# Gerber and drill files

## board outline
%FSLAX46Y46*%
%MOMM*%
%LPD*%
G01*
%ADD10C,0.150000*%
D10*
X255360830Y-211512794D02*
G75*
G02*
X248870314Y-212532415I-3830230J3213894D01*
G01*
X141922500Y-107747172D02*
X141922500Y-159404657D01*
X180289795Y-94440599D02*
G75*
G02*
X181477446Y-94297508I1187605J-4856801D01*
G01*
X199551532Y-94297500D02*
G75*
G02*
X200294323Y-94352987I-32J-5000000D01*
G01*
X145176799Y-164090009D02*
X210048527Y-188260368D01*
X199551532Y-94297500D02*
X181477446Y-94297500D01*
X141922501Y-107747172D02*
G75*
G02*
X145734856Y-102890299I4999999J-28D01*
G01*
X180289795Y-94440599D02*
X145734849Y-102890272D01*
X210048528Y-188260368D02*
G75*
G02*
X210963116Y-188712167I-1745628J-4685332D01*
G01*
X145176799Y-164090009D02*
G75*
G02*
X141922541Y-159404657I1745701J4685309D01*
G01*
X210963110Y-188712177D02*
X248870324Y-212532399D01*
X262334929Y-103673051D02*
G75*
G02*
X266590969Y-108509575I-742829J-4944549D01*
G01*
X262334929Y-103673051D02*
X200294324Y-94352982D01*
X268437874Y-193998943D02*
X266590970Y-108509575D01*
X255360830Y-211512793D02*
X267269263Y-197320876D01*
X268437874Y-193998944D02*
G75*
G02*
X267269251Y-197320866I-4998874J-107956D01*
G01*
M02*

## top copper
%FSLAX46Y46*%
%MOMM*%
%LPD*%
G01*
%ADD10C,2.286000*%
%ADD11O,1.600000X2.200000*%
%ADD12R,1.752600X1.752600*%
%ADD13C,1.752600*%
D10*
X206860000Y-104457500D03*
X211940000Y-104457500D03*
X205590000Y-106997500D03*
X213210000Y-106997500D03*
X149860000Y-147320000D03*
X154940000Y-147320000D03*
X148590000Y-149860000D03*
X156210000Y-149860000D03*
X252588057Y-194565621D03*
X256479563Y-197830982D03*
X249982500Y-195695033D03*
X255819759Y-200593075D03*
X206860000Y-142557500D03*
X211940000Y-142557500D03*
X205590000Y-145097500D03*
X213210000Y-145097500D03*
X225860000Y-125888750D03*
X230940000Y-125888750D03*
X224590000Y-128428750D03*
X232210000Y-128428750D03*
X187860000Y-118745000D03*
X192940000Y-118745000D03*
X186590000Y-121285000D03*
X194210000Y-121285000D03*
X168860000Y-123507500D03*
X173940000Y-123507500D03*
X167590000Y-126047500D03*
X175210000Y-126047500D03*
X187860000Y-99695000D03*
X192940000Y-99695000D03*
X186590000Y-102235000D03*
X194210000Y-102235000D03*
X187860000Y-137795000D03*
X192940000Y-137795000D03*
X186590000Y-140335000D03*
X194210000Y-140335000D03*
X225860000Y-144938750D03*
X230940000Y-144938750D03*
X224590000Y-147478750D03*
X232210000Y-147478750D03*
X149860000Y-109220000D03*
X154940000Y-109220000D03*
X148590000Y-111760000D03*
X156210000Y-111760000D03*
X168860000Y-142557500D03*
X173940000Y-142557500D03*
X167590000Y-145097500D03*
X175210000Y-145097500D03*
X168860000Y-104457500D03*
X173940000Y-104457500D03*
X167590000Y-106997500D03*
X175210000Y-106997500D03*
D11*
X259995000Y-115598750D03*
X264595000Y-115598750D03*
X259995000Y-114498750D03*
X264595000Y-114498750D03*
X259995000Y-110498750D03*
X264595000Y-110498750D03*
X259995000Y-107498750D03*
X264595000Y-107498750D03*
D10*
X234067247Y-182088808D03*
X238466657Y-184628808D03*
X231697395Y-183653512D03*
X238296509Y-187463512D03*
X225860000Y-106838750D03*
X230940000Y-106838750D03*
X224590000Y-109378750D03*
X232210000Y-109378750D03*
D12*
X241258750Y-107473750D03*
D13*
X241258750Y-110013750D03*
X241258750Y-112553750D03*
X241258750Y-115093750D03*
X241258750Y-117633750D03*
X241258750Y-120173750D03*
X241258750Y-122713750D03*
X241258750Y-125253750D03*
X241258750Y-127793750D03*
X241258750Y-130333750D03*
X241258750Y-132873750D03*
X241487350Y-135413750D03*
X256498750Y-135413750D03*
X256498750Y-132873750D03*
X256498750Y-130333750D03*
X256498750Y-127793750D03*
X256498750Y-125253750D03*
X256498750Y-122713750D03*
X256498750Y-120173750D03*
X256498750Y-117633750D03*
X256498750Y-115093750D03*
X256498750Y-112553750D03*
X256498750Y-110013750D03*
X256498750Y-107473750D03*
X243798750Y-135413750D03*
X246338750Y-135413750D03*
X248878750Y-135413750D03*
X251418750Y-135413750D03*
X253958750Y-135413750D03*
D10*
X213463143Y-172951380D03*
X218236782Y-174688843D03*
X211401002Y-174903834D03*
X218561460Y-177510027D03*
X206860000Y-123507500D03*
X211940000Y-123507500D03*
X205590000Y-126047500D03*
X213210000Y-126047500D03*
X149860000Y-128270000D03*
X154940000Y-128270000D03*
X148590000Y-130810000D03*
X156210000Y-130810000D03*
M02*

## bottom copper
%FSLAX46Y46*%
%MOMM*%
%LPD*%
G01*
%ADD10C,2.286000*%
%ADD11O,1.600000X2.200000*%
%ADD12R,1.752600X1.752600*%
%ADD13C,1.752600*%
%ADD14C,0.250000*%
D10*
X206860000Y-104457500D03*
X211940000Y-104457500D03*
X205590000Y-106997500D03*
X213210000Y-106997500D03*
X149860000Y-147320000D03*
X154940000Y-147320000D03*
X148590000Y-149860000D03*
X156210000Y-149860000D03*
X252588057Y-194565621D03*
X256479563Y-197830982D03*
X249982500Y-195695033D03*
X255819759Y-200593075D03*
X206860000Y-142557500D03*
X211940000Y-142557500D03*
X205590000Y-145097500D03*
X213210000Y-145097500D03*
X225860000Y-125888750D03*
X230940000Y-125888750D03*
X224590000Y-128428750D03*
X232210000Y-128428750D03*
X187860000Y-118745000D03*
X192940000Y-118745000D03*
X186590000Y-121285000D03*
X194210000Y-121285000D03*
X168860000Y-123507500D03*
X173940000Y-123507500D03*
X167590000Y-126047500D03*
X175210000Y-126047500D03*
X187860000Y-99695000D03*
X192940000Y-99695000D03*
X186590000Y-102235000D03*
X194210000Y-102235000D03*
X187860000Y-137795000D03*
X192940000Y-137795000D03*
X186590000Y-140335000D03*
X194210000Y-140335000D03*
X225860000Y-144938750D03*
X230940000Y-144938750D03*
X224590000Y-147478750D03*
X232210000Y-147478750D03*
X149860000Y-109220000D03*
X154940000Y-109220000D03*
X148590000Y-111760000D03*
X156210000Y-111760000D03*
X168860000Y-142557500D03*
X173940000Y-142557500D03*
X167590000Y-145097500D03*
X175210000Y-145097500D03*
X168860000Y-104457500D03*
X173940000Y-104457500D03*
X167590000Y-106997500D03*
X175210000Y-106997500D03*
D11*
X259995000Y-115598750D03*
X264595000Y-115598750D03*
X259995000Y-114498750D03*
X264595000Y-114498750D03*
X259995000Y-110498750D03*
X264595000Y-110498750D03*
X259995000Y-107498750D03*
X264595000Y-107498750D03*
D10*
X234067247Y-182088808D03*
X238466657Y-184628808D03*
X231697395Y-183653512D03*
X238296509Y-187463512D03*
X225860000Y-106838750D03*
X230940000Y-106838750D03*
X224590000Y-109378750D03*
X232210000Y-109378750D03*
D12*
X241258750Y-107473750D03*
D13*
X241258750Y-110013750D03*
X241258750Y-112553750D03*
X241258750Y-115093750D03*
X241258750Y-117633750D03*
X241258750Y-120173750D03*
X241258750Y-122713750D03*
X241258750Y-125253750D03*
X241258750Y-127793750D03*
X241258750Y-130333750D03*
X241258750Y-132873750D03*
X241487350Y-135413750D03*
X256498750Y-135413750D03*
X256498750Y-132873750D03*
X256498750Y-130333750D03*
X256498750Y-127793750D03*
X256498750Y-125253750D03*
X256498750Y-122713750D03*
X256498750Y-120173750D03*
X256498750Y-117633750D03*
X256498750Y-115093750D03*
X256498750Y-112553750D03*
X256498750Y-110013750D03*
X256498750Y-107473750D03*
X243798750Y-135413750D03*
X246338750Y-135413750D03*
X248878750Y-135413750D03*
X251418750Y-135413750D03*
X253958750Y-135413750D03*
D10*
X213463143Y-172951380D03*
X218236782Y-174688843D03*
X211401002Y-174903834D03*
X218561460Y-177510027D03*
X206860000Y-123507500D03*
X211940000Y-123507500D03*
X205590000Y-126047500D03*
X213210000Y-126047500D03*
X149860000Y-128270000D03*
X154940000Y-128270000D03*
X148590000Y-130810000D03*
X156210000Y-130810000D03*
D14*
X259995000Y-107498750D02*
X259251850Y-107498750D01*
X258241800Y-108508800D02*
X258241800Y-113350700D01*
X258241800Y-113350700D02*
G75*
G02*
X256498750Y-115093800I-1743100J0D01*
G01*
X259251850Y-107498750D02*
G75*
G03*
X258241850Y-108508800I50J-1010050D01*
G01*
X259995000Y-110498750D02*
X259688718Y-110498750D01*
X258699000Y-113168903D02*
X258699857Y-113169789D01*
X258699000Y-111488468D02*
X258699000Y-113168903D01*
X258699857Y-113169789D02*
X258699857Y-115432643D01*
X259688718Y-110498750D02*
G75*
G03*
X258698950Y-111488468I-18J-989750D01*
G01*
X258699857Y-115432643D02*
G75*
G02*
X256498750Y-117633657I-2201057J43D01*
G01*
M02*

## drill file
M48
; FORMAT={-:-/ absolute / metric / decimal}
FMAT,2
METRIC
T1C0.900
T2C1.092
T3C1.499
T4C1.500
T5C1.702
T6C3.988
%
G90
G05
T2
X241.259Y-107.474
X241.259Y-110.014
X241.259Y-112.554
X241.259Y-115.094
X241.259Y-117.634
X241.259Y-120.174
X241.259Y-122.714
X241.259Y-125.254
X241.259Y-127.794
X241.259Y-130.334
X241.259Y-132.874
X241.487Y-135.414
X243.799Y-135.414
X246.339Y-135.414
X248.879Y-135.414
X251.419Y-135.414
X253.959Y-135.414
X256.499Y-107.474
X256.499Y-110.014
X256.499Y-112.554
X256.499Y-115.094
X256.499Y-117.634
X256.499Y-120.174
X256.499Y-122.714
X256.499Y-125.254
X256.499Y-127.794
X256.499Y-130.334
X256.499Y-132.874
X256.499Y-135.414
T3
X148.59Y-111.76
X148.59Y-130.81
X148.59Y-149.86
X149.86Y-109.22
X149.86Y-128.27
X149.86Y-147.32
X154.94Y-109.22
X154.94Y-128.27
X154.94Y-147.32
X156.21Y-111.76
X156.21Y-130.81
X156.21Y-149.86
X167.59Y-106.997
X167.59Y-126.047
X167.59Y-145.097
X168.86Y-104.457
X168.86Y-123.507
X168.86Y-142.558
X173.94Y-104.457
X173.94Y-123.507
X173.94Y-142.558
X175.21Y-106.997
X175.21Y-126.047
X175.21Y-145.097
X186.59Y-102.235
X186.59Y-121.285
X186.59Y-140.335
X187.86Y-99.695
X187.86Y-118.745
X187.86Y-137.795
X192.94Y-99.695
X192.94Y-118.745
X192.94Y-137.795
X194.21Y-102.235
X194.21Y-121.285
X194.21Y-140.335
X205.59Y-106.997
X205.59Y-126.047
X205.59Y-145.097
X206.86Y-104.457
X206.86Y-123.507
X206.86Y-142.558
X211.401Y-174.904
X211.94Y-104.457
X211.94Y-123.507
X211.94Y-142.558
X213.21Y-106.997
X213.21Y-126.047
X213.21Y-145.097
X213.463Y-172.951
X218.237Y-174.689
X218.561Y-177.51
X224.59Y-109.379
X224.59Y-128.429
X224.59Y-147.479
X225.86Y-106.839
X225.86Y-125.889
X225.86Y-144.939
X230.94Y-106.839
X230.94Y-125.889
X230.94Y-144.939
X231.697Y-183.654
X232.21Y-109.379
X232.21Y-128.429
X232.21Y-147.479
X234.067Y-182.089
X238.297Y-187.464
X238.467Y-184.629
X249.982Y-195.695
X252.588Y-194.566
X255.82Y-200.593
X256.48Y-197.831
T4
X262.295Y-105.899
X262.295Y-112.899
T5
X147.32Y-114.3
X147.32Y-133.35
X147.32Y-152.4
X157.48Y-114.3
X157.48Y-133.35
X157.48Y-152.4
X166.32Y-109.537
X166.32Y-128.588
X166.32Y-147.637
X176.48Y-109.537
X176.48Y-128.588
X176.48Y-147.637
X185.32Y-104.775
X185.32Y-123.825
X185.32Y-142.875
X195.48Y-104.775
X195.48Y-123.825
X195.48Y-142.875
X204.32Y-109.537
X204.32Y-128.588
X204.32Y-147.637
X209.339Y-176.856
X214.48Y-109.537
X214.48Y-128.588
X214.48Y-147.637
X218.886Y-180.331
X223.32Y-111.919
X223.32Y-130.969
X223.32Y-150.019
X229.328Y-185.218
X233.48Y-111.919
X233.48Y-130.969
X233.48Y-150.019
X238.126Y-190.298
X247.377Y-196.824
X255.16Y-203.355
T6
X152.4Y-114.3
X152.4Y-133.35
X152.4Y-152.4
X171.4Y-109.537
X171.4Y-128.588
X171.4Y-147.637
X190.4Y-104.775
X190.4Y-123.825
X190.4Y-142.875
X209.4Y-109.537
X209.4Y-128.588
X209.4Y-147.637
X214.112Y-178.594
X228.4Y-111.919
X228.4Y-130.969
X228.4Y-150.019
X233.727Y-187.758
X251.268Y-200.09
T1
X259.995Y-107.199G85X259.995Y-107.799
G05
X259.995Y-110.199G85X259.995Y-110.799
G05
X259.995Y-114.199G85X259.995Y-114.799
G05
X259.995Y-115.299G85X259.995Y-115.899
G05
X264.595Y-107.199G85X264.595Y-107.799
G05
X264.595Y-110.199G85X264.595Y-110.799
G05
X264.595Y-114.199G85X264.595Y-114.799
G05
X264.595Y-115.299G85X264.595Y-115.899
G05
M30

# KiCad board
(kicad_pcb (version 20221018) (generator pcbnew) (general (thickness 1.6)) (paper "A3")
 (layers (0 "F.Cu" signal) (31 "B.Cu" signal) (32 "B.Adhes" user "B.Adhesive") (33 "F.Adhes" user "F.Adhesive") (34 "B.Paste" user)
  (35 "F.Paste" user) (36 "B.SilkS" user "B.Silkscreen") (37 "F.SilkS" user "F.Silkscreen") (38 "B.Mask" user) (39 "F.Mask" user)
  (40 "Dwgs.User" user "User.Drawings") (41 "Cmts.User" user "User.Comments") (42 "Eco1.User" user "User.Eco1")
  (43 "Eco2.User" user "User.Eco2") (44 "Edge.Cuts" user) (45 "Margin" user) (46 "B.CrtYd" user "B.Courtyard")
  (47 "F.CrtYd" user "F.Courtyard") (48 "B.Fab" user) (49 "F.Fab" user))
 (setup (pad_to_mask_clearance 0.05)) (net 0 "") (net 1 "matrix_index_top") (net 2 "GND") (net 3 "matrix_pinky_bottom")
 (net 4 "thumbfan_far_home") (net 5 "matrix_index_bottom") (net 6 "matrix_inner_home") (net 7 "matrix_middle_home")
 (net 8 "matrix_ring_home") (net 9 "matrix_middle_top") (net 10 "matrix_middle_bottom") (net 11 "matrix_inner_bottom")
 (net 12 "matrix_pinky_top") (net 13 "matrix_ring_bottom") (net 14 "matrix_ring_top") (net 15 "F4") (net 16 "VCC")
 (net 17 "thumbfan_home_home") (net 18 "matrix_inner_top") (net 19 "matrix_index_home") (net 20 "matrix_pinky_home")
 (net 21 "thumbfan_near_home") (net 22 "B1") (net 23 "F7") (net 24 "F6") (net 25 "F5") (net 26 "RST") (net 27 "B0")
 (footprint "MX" (layer "F.Cu") (at 209.4 109.5375)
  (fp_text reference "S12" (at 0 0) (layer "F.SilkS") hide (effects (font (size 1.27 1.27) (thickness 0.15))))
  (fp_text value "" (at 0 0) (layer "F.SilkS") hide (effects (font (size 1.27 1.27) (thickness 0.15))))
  (pad "" np_thru_hole circle (at -5.08 0) (size 1.7018 1.7018) (drill 1.7018) (layers "*.Cu" "*.Mask"))
  (pad "" np_thru_hole circle (at 0 0) (size 3.9878 3.9878) (drill 3.9878) (layers "*.Cu" "*.Mask"))
  (pad "" np_thru_hole circle (at 5.08 0) (size 1.7018 1.7018) (drill 1.7018) (layers "*.Cu" "*.Mask"))
  (pad "1" thru_hole circle (at -2.54 -5.08) (size 2.286 2.286) (drill 1.4986) (layers "*.Cu" "*.Mask") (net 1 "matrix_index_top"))
  (pad "1" thru_hole circle (at 2.54 -5.08) (size 2.286 2.286) (drill 1.4986) (layers "*.Cu" "*.Mask") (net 1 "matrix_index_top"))
  (pad "2" thru_hole circle (at -3.81 -2.54) (size 2.286 2.286) (drill 1.4986) (layers "*.Cu" "*.Mask") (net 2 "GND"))
  (pad "2" thru_hole circle (at 3.81 -2.54) (size 2.286 2.286) (drill 1.4986) (layers "*.Cu" "*.Mask") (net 2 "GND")))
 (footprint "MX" (layer "F.Cu") (at 152.4 152.4)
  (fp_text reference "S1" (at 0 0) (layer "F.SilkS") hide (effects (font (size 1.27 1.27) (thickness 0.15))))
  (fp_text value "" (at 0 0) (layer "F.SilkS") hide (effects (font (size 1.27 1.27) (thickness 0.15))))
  (pad "" np_thru_hole circle (at -5.08 0) (size 1.7018 1.7018) (drill 1.7018) (layers "*.Cu" "*.Mask"))
  (pad "" np_thru_hole circle (at 0 0) (size 3.9878 3.9878) (drill 3.9878) (layers "*.Cu" "*.Mask"))
  (pad "" np_thru_hole circle (at 5.08 0) (size 1.7018 1.7018) (drill 1.7018) (layers "*.Cu" "*.Mask"))
  (pad "1" thru_hole circle (at -2.54 -5.08) (size 2.286 2.286) (drill 1.4986) (layers "*.Cu" "*.Mask") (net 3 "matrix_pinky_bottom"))
  (pad "1" thru_hole circle (at 2.54 -5.08) (size 2.286 2.286) (drill 1.4986) (layers "*.Cu" "*.Mask") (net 3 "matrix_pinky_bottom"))
  (pad "2" thru_hole circle (at -3.81 -2.54) (size 2.286 2.286) (drill 1.4986) (layers "*.Cu" "*.Mask") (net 2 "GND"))
  (pad "2" thru_hole circle (at 3.81 -2.54) (size 2.286 2.286) (drill 1.4986) (layers "*.Cu" "*.Mask") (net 2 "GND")))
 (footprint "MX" (layer "F.Cu") (at 251.268449 200.089807 -40)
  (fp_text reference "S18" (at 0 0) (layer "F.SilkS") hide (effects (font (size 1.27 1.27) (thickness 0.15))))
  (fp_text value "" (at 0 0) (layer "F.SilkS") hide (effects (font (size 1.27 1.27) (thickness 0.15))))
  (pad "" np_thru_hole circle (at -5.08 0) (size 1.7018 1.7018) (drill 1.7018) (layers "*.Cu" "*.Mask"))
  (pad "" np_thru_hole circle (at 0 0) (size 3.9878 3.9878) (drill 3.9878) (layers "*.Cu" "*.Mask"))
  (pad "" np_thru_hole circle (at 5.08 0) (size 1.7018 1.7018) (drill 1.7018) (layers "*.Cu" "*.Mask"))
  (pad "1" thru_hole circle (at -2.54 -5.08) (size 2.286 2.286) (drill 1.4986) (layers "*.Cu" "*.Mask") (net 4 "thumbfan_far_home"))
  (pad "1" thru_hole circle (at 2.54 -5.08) (size 2.286 2.286) (drill 1.4986) (layers "*.Cu" "*.Mask") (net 4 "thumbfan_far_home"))
  (pad "2" thru_hole circle (at -3.81 -2.54) (size 2.286 2.286) (drill 1.4986) (layers "*.Cu" "*.Mask") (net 2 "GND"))
  (pad "2" thru_hole circle (at 3.81 -2.54) (size 2.286 2.286) (drill 1.4986) (layers "*.Cu" "*.Mask") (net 2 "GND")))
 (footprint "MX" (layer "F.Cu") (at 209.4 147.6375)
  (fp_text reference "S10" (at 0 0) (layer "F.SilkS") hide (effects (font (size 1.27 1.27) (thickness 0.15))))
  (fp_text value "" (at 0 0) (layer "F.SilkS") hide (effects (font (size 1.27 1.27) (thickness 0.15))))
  (pad "" np_thru_hole circle (at -5.08 0) (size 1.7018 1.7018) (drill 1.7018) (layers "*.Cu" "*.Mask"))
  (pad "" np_thru_hole circle (at 0 0) (size 3.9878 3.9878) (drill 3.9878) (layers "*.Cu" "*.Mask"))
  (pad "" np_thru_hole circle (at 5.08 0) (size 1.7018 1.7018) (drill 1.7018) (layers "*.Cu" "*.Mask"))
  (pad "1" thru_hole circle (at -2.54 -5.08) (size 2.286 2.286) (drill 1.4986) (layers "*.Cu" "*.Mask") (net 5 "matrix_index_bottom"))
  (pad "1" thru_hole circle (at 2.54 -5.08) (size 2.286 2.286) (drill 1.4986) (layers "*.Cu" "*.Mask") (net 5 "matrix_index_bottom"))
  (pad "2" thru_hole circle (at -3.81 -2.54) (size 2.286 2.286) (drill 1.4986) (layers "*.Cu" "*.Mask") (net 2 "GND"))
  (pad "2" thru_hole circle (at 3.81 -2.54) (size 2.286 2.286) (drill 1.4986) (layers "*.Cu" "*.Mask") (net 2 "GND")))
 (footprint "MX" (layer "F.Cu") (at 228.4 130.96875)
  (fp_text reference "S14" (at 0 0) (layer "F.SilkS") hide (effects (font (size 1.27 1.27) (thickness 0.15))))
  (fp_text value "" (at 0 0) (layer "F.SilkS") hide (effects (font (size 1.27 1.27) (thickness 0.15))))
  (pad "" np_thru_hole circle (at -5.08 0) (size 1.7018 1.7018) (drill 1.7018) (layers "*.Cu" "*.Mask"))
  (pad "" np_thru_hole circle (at 0 0) (size 3.9878 3.9878) (drill 3.9878) (layers "*.Cu" "*.Mask"))
  (pad "" np_thru_hole circle (at 5.08 0) (size 1.7018 1.7018) (drill 1.7018) (layers "*.Cu" "*.Mask"))
  (pad "1" thru_hole circle (at -2.54 -5.08) (size 2.286 2.286) (drill 1.4986) (layers "*.Cu" "*.Mask") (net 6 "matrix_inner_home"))
  (pad "1" thru_hole circle (at 2.54 -5.08) (size 2.286 2.286) (drill 1.4986) (layers "*.Cu" "*.Mask") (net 6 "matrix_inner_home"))
  (pad "2" thru_hole circle (at -3.81 -2.54) (size 2.286 2.286) (drill 1.4986) (layers "*.Cu" "*.Mask") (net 2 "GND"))
  (pad "2" thru_hole circle (at 3.81 -2.54) (size 2.286 2.286) (drill 1.4986) (layers "*.Cu" "*.Mask") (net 2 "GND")))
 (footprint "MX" (layer "F.Cu") (at 190.4 123.825)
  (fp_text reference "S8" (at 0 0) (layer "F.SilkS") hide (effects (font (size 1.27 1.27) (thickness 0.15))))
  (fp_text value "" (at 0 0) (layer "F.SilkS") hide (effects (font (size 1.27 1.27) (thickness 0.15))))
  (pad "" np_thru_hole circle (at -5.08 0) (size 1.7018 1.7018) (drill 1.7018) (layers "*.Cu" "*.Mask"))
  (pad "" np_thru_hole circle (at 0 0) (size 3.9878 3.9878) (drill 3.9878) (layers "*.Cu" "*.Mask"))
  (pad "" np_thru_hole circle (at 5.08 0) (size 1.7018 1.7018) (drill 1.7018) (layers "*.Cu" "*.Mask"))
  (pad "1" thru_hole circle (at -2.54 -5.08) (size 2.286 2.286) (drill 1.4986) (layers "*.Cu" "*.Mask") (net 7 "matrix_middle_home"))
  (pad "1" thru_hole circle (at 2.54 -5.08) (size 2.286 2.286) (drill 1.4986) (layers "*.Cu" "*.Mask") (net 7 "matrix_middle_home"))
  (pad "2" thru_hole circle (at -3.81 -2.54) (size 2.286 2.286) (drill 1.4986) (layers "*.Cu" "*.Mask") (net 2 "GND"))
  (pad "2" thru_hole circle (at 3.81 -2.54) (size 2.286 2.286) (drill 1.4986) (layers "*.Cu" "*.Mask") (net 2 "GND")))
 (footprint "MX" (layer "F.Cu") (at 171.4 128.5875)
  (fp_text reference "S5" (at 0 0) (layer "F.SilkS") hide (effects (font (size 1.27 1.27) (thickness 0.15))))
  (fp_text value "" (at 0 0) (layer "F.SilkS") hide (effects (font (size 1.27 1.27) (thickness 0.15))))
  (pad "" np_thru_hole circle (at -5.08 0) (size 1.7018 1.7018) (drill 1.7018) (layers "*.Cu" "*.Mask"))
  (pad "" np_thru_hole circle (at 0 0) (size 3.9878 3.9878) (drill 3.9878) (layers "*.Cu" "*.Mask"))
  (pad "" np_thru_hole circle (at 5.08 0) (size 1.7018 1.7018) (drill 1.7018) (layers "*.Cu" "*.Mask"))
  (pad "1" thru_hole circle (at -2.54 -5.08) (size 2.286 2.286) (drill 1.4986) (layers "*.Cu" "*.Mask") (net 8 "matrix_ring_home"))
  (pad "1" thru_hole circle (at 2.54 -5.08) (size 2.286 2.286) (drill 1.4986) (layers "*.Cu" "*.Mask") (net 8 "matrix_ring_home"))
  (pad "2" thru_hole circle (at -3.81 -2.54) (size 2.286 2.286) (drill 1.4986) (layers "*.Cu" "*.Mask") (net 2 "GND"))
  (pad "2" thru_hole circle (at 3.81 -2.54) (size 2.286 2.286) (drill 1.4986) (layers "*.Cu" "*.Mask") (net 2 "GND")))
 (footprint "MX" (layer "F.Cu") (at 190.4 104.775)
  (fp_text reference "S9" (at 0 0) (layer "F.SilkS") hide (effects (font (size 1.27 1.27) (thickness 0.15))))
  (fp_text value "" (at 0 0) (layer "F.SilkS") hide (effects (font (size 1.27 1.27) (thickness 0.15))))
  (pad "" np_thru_hole circle (at -5.08 0) (size 1.7018 1.7018) (drill 1.7018) (layers "*.Cu" "*.Mask"))
  (pad "" np_thru_hole circle (at 0 0) (size 3.9878 3.9878) (drill 3.9878) (layers "*.Cu" "*.Mask"))
  (pad "" np_thru_hole circle (at 5.08 0) (size 1.7018 1.7018) (drill 1.7018) (layers "*.Cu" "*.Mask"))
  (pad "1" thru_hole circle (at -2.54 -5.08) (size 2.286 2.286) (drill 1.4986) (layers "*.Cu" "*.Mask") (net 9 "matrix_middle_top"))
  (pad "1" thru_hole circle (at 2.54 -5.08) (size 2.286 2.286) (drill 1.4986) (layers "*.Cu" "*.Mask") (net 9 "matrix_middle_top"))
  (pad "2" thru_hole circle (at -3.81 -2.54) (size 2.286 2.286) (drill 1.4986) (layers "*.Cu" "*.Mask") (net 2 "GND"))
  (pad "2" thru_hole circle (at 3.81 -2.54) (size 2.286 2.286) (drill 1.4986) (layers "*.Cu" "*.Mask") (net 2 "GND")))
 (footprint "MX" (layer "F.Cu") (at 190.4 142.875)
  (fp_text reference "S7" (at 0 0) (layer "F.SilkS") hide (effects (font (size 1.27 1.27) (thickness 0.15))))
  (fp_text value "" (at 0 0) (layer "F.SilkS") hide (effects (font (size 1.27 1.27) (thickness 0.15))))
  (pad "" np_thru_hole circle (at -5.08 0) (size 1.7018 1.7018) (drill 1.7018) (layers "*.Cu" "*.Mask"))
  (pad "" np_thru_hole circle (at 0 0) (size 3.9878 3.9878) (drill 3.9878) (layers "*.Cu" "*.Mask"))
  (pad "" np_thru_hole circle (at 5.08 0) (size 1.7018 1.7018) (drill 1.7018) (layers "*.Cu" "*.Mask"))
  (pad "1" thru_hole circle (at -2.54 -5.08) (size 2.286 2.286) (drill 1.4986) (layers "*.Cu" "*.Mask") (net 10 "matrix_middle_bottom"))
  (pad "1" thru_hole circle (at 2.54 -5.08) (size 2.286 2.286) (drill 1.4986) (layers "*.Cu" "*.Mask") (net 10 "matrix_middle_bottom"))
  (pad "2" thru_hole circle (at -3.81 -2.54) (size 2.286 2.286) (drill 1.4986) (layers "*.Cu" "*.Mask") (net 2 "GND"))
  (pad "2" thru_hole circle (at 3.81 -2.54) (size 2.286 2.286) (drill 1.4986) (layers "*.Cu" "*.Mask") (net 2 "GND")))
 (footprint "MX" (layer "F.Cu") (at 228.4 150.01875)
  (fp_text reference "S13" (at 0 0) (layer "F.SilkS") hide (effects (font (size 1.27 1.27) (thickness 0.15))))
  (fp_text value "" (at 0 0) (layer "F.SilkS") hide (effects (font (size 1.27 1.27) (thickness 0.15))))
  (pad "" np_thru_hole circle (at -5.08 0) (size 1.7018 1.7018) (drill 1.7018) (layers "*.Cu" "*.Mask"))
  (pad "" np_thru_hole circle (at 0 0) (size 3.9878 3.9878) (drill 3.9878) (layers "*.Cu" "*.Mask"))
  (pad "" np_thru_hole circle (at 5.08 0) (size 1.7018 1.7018) (drill 1.7018) (layers "*.Cu" "*.Mask"))
  (pad "1" thru_hole circle (at -2.54 -5.08) (size 2.286 2.286) (drill 1.4986) (layers "*.Cu" "*.Mask") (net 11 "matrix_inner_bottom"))
  (pad "1" thru_hole circle (at 2.54 -5.08) (size 2.286 2.286) (drill 1.4986) (layers "*.Cu" "*.Mask") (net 11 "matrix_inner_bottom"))
  (pad "2" thru_hole circle (at -3.81 -2.54) (size 2.286 2.286) (drill 1.4986) (layers "*.Cu" "*.Mask") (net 2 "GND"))
  (pad "2" thru_hole circle (at 3.81 -2.54) (size 2.286 2.286) (drill 1.4986) (layers "*.Cu" "*.Mask") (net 2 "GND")))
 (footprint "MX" (layer "F.Cu") (at 152.4 114.3)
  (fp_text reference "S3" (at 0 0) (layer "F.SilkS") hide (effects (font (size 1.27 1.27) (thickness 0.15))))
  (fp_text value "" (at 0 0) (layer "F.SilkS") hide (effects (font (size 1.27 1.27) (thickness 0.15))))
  (pad "" np_thru_hole circle (at -5.08 0) (size 1.7018 1.7018) (drill 1.7018) (layers "*.Cu" "*.Mask"))
  (pad "" np_thru_hole circle (at 0 0) (size 3.9878 3.9878) (drill 3.9878) (layers "*.Cu" "*.Mask"))
  (pad "" np_thru_hole circle (at 5.08 0) (size 1.7018 1.7018) (drill 1.7018) (layers "*.Cu" "*.Mask"))
  (pad "1" thru_hole circle (at -2.54 -5.08) (size 2.286 2.286) (drill 1.4986) (layers "*.Cu" "*.Mask") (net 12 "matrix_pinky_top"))
  (pad "1" thru_hole circle (at 2.54 -5.08) (size 2.286 2.286) (drill 1.4986) (layers "*.Cu" "*.Mask") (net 12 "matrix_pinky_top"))
  (pad "2" thru_hole circle (at -3.81 -2.54) (size 2.286 2.286) (drill 1.4986) (layers "*.Cu" "*.Mask") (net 2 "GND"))
  (pad "2" thru_hole circle (at 3.81 -2.54) (size 2.286 2.286) (drill 1.4986) (layers "*.Cu" "*.Mask") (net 2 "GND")))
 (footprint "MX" (layer "F.Cu") (at 171.4 147.6375)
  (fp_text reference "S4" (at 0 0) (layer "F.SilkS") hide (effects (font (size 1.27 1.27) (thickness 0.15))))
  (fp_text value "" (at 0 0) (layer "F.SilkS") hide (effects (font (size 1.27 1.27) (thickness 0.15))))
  (pad "" np_thru_hole circle (at -5.08 0) (size 1.7018 1.7018) (drill 1.7018) (layers "*.Cu" "*.Mask"))
  (pad "" np_thru_hole circle (at 0 0) (size 3.9878 3.9878) (drill 3.9878) (layers "*.Cu" "*.Mask"))
  (pad "" np_thru_hole circle (at 5.08 0) (size 1.7018 1.7018) (drill 1.7018) (layers "*.Cu" "*.Mask"))
  (pad "1" thru_hole circle (at -2.54 -5.08) (size 2.286 2.286) (drill 1.4986) (layers "*.Cu" "*.Mask") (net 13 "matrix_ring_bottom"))
  (pad "1" thru_hole circle (at 2.54 -5.08) (size 2.286 2.286) (drill 1.4986) (layers "*.Cu" "*.Mask") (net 13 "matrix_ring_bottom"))
  (pad "2" thru_hole circle (at -3.81 -2.54) (size 2.286 2.286) (drill 1.4986) (layers "*.Cu" "*.Mask") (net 2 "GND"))
  (pad "2" thru_hole circle (at 3.81 -2.54) (size 2.286 2.286) (drill 1.4986) (layers "*.Cu" "*.Mask") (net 2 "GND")))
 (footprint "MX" (layer "F.Cu") (at 171.4 109.5375)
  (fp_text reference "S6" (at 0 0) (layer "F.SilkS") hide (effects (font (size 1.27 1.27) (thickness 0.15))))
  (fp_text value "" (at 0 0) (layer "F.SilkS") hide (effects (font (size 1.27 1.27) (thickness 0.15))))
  (pad "" np_thru_hole circle (at -5.08 0) (size 1.7018 1.7018) (drill 1.7018) (layers "*.Cu" "*.Mask"))
  (pad "" np_thru_hole circle (at 0 0) (size 3.9878 3.9878) (drill 3.9878) (layers "*.Cu" "*.Mask"))
  (pad "" np_thru_hole circle (at 5.08 0) (size 1.7018 1.7018) (drill 1.7018) (layers "*.Cu" "*.Mask"))
  (pad "1" thru_hole circle (at -2.54 -5.08) (size 2.286 2.286) (drill 1.4986) (layers "*.Cu" "*.Mask") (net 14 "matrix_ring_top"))
  (pad "1" thru_hole circle (at 2.54 -5.08) (size 2.286 2.286) (drill 1.4986) (layers "*.Cu" "*.Mask") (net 14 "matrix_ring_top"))
  (pad "2" thru_hole circle (at -3.81 -2.54) (size 2.286 2.286) (drill 1.4986) (layers "*.Cu" "*.Mask") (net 2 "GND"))
  (pad "2" thru_hole circle (at 3.81 -2.54) (size 2.286 2.286) (drill 1.4986) (layers "*.Cu" "*.Mask") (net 2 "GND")))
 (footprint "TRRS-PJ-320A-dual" (layer "F.Cu") (at 264.595 104.29875)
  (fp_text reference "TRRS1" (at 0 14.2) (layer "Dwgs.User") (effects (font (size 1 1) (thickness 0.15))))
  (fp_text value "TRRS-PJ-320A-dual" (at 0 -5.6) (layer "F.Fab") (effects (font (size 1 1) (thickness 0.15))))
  (pad "" np_thru_hole circle (at -2.3 1.6) (size 1.5 1.5) (drill 1.5) (layers "*.Cu" "*.Mask"))
  (pad "" np_thru_hole circle (at -2.3 8.6) (size 1.5 1.5) (drill 1.5) (layers "*.Cu" "*.Mask"))
  (pad "1" thru_hole oval (at -4.6 11.3) (size 1.6 2.2) (drill oval 0.9 1.5) (layers "*.Cu" "*.Mask") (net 2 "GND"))
  (pad "1" thru_hole oval (at 0 11.3) (size 1.6 2.2) (drill oval 0.9 1.5) (layers "*.Cu" "*.Mask") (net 2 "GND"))
  (pad "2" thru_hole oval (at -4.6 10.2) (size 1.6 2.2) (drill oval 0.9 1.5) (layers "*.Cu" "*.Mask") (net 2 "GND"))
  (pad "2" thru_hole oval (at 0 10.2) (size 1.6 2.2) (drill oval 0.9 1.5) (layers "*.Cu" "*.Mask") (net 2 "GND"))
  (pad "3" thru_hole oval (at -4.6 6.2) (size 1.6 2.2) (drill oval 0.9 1.5) (layers "*.Cu" "*.Mask") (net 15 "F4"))
  (pad "3" thru_hole oval (at 0 6.2) (size 1.6 2.2) (drill oval 0.9 1.5) (layers "*.Cu" "*.Mask") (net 15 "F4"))
  (pad "4" thru_hole oval (at -4.6 3.2) (size 1.6 2.2) (drill oval 0.9 1.5) (layers "*.Cu" "*.Mask") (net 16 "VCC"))
  (pad "4" thru_hole oval (at 0 3.2) (size 1.6 2.2) (drill oval 0.9 1.5) (layers "*.Cu" "*.Mask") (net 16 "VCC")))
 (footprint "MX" (layer "F.Cu") (at 233.726952 187.758217 -30)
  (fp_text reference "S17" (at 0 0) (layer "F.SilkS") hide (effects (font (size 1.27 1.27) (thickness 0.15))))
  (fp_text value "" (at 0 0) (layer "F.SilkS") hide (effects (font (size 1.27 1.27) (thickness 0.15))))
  (pad "" np_thru_hole circle (at -5.08 0) (size 1.7018 1.7018) (drill 1.7018) (layers "*.Cu" "*.Mask"))
  (pad "" np_thru_hole circle (at 0 0) (size 3.9878 3.9878) (drill 3.9878) (layers "*.Cu" "*.Mask"))
  (pad "" np_thru_hole circle (at 5.08 0) (size 1.7018 1.7018) (drill 1.7018) (layers "*.Cu" "*.Mask"))
  (pad "1" thru_hole circle (at -2.54 -5.08) (size 2.286 2.286) (drill 1.4986) (layers "*.Cu" "*.Mask") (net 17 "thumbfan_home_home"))
  (pad "1" thru_hole circle (at 2.54 -5.08) (size 2.286 2.286) (drill 1.4986) (layers "*.Cu" "*.Mask") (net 17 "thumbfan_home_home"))
  (pad "2" thru_hole circle (at -3.81 -2.54) (size 2.286 2.286) (drill 1.4986) (layers "*.Cu" "*.Mask") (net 2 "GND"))
  (pad "2" thru_hole circle (at 3.81 -2.54) (size 2.286 2.286) (drill 1.4986) (layers "*.Cu" "*.Mask") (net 2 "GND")))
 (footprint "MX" (layer "F.Cu") (at 228.4 111.91875)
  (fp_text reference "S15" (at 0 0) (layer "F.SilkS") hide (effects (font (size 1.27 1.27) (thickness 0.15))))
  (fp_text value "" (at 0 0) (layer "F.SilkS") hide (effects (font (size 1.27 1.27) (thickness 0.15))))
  (pad "" np_thru_hole circle (at -5.08 0) (size 1.7018 1.7018) (drill 1.7018) (layers "*.Cu" "*.Mask"))
  (pad "" np_thru_hole circle (at 0 0) (size 3.9878 3.9878) (drill 3.9878) (layers "*.Cu" "*.Mask"))
  (pad "" np_thru_hole circle (at 5.08 0) (size 1.7018 1.7018) (drill 1.7018) (layers "*.Cu" "*.Mask"))
  (pad "1" thru_hole circle (at -2.54 -5.08) (size 2.286 2.286) (drill 1.4986) (layers "*.Cu" "*.Mask") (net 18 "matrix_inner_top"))
  (pad "1" thru_hole circle (at 2.54 -5.08) (size 2.286 2.286) (drill 1.4986) (layers "*.Cu" "*.Mask") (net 18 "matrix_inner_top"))
  (pad "2" thru_hole circle (at -3.81 -2.54) (size 2.286 2.286) (drill 1.4986) (layers "*.Cu" "*.Mask") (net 2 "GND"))
  (pad "2" thru_hole circle (at 3.81 -2.54) (size 2.286 2.286) (drill 1.4986) (layers "*.Cu" "*.Mask") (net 2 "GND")))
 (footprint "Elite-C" (layer "F.Cu") (at 248.87875 121.44375 -90)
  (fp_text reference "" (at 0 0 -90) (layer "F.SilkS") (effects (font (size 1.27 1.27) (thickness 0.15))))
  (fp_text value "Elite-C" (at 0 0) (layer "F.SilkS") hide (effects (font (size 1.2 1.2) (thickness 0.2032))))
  (pad "1" thru_hole rect (at -13.97 7.62) (size 1.7526 1.7526) (drill 1.0922) (layers "*.Cu" "*.SilkS" "*.Mask")
   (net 18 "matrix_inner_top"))
  (pad "2" thru_hole circle (at -11.43 7.62) (size 1.7526 1.7526) (drill 1.0922) (layers "*.Cu" "*.SilkS" "*.Mask")
   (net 1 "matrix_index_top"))
  (pad "3" thru_hole circle (at -8.89 7.62) (size 1.7526 1.7526) (drill 1.0922) (layers "*.Cu" "*.SilkS" "*.Mask") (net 2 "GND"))
  (pad "4" thru_hole circle (at -6.35 7.62) (size 1.7526 1.7526) (drill 1.0922) (layers "*.Cu" "*.SilkS" "*.Mask") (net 2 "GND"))
  (pad "5" thru_hole circle (at -3.81 7.62) (size 1.7526 1.7526) (drill 1.0922) (layers "*.Cu" "*.SilkS" "*.Mask")
   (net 9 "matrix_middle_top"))
  (pad "6" thru_hole circle (at -1.27 7.62) (size 1.7526 1.7526) (drill 1.0922) (layers "*.Cu" "*.SilkS" "*.Mask")
   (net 14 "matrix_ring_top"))
  (pad "7" thru_hole circle (at 1.27 7.62) (size 1.7526 1.7526) (drill 1.0922) (layers "*.Cu" "*.SilkS" "*.Mask")
   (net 12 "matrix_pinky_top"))
  (pad "8" thru_hole circle (at 3.81 7.62) (size 1.7526 1.7526) (drill 1.0922) (layers "*.Cu" "*.SilkS" "*.Mask")
   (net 7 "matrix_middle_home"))
  (pad "9" thru_hole circle (at 6.35 7.62) (size 1.7526 1.7526) (drill 1.0922) (layers "*.Cu" "*.SilkS" "*.Mask")
   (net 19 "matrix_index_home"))
  (pad "10" thru_hole circle (at 8.89 7.62) (size 1.7526 1.7526) (drill 1.0922) (layers "*.Cu" "*.SilkS" "*.Mask")
   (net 6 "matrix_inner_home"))
  (pad "11" thru_hole circle (at 11.43 7.62) (size 1.7526 1.7526) (drill 1.0922) (layers "*.Cu" "*.SilkS" "*.Mask")
   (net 8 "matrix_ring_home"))
  (pad "12" thru_hole circle (at 13.97 7.3914) (size 1.7526 1.7526) (drill 1.0922) (layers "*.Cu" "*.SilkS" "*.Mask")
   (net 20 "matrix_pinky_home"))
  (pad "13" thru_hole circle (at 13.97 -7.62) (size 1.7526 1.7526) (drill 1.0922) (layers "*.Cu" "*.SilkS" "*.Mask")
   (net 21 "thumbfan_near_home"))
  (pad "14" thru_hole circle (at 11.43 -7.62) (size 1.7526 1.7526) (drill 1.0922) (layers "*.Cu" "*.SilkS" "*.Mask")
   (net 17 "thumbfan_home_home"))
  (pad "15" thru_hole circle (at 8.89 -7.62) (size 1.7526 1.7526) (drill 1.0922) (layers "*.Cu" "*.SilkS" "*.Mask")
   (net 4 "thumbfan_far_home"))
  (pad "16" thru_hole circle (at 6.35 -7.62) (size 1.7526 1.7526) (drill 1.0922) (layers "*.Cu" "*.SilkS" "*.Mask") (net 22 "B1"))
  (pad "17" thru_hole circle (at 3.81 -7.62) (size 1.7526 1.7526) (drill 1.0922) (layers "*.Cu" "*.SilkS" "*.Mask") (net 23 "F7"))
  (pad "18" thru_hole circle (at 1.27 -7.62) (size 1.7526 1.7526) (drill 1.0922) (layers "*.Cu" "*.SilkS" "*.Mask") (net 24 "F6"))
  (pad "19" thru_hole circle (at -1.27 -7.62) (size 1.7526 1.7526) (drill 1.0922) (layers "*.Cu" "*.SilkS" "*.Mask") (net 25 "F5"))
  (pad "20" thru_hole circle (at -3.81 -7.62) (size 1.7526 1.7526) (drill 1.0922) (layers "*.Cu" "*.SilkS" "*.Mask") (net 15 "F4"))
  (pad "21" thru_hole circle (at -6.35 -7.62) (size 1.7526 1.7526) (drill 1.0922) (layers "*.Cu" "*.SilkS" "*.Mask") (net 16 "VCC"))
  (pad "22" thru_hole circle (at -8.89 -7.62) (size 1.7526 1.7526) (drill 1.0922) (layers "*.Cu" "*.SilkS" "*.Mask") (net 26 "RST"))
  (pad "23" thru_hole circle (at -11.43 -7.62) (size 1.7526 1.7526) (drill 1.0922) (layers "*.Cu" "*.SilkS" "*.Mask") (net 2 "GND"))
  (pad "24" thru_hole circle (at -13.97 -7.62) (size 1.7526 1.7526) (drill 1.0922) (layers "*.Cu" "*.SilkS" "*.Mask") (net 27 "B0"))
  (pad "25" thru_hole circle (at 13.97 5.08) (size 1.7526 1.7526) (drill 1.0922) (layers "*.Cu" "*.SilkS" "*.Mask")
   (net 10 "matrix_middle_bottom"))
  (pad "26" thru_hole circle (at 13.97 2.54) (size 1.7526 1.7526) (drill 1.0922) (layers "*.Cu" "*.SilkS" "*.Mask")
   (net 5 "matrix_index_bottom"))
  (pad "27" thru_hole circle (at 13.97 0) (size 1.7526 1.7526) (drill 1.0922) (layers "*.Cu" "*.SilkS" "*.Mask")
   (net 11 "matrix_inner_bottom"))
  (pad "28" thru_hole circle (at 13.97 -2.54) (size 1.7526 1.7526) (drill 1.0922) (layers "*.Cu" "*.SilkS" "*.Mask")
   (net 3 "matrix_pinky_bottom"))
  (pad "29" thru_hole circle (at 13.97 -5.08) (size 1.7526 1.7526) (drill 1.0922) (layers "*.Cu" "*.SilkS" "*.Mask")
   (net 13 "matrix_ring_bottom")))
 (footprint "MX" (layer "F.Cu") (at 214.1125 178.59375 -20)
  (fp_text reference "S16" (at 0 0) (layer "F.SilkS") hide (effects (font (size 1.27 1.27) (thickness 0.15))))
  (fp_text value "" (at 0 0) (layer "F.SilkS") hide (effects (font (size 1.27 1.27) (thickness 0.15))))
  (pad "" np_thru_hole circle (at -5.08 0) (size 1.7018 1.7018) (drill 1.7018) (layers "*.Cu" "*.Mask"))
  (pad "" np_thru_hole circle (at 0 0) (size 3.9878 3.9878) (drill 3.9878) (layers "*.Cu" "*.Mask"))
  (pad "" np_thru_hole circle (at 5.08 0) (size 1.7018 1.7018) (drill 1.7018) (layers "*.Cu" "*.Mask"))
  (pad "1" thru_hole circle (at -2.54 -5.08) (size 2.286 2.286) (drill 1.4986) (layers "*.Cu" "*.Mask") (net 21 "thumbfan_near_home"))
  (pad "1" thru_hole circle (at 2.54 -5.08) (size 2.286 2.286) (drill 1.4986) (layers "*.Cu" "*.Mask") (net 21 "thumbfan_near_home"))
  (pad "2" thru_hole circle (at -3.81 -2.54) (size 2.286 2.286) (drill 1.4986) (layers "*.Cu" "*.Mask") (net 2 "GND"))
  (pad "2" thru_hole circle (at 3.81 -2.54) (size 2.286 2.286) (drill 1.4986) (layers "*.Cu" "*.Mask") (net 2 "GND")))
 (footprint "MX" (layer "F.Cu") (at 209.4 128.5875)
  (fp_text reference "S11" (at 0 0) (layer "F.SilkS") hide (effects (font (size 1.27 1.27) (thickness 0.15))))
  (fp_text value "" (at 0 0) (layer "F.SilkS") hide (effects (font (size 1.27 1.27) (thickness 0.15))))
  (pad "" np_thru_hole circle (at -5.08 0) (size 1.7018 1.7018) (drill 1.7018) (layers "*.Cu" "*.Mask"))
  (pad "" np_thru_hole circle (at 0 0) (size 3.9878 3.9878) (drill 3.9878) (layers "*.Cu" "*.Mask"))
  (pad "" np_thru_hole circle (at 5.08 0) (size 1.7018 1.7018) (drill 1.7018) (layers "*.Cu" "*.Mask"))
  (pad "1" thru_hole circle (at -2.54 -5.08) (size 2.286 2.286) (drill 1.4986) (layers "*.Cu" "*.Mask") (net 19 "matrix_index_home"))
  (pad "1" thru_hole circle (at 2.54 -5.08) (size 2.286 2.286) (drill 1.4986) (layers "*.Cu" "*.Mask") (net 19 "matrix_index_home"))
  (pad "2" thru_hole circle (at -3.81 -2.54) (size 2.286 2.286) (drill 1.4986) (layers "*.Cu" "*.Mask") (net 2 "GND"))
  (pad "2" thru_hole circle (at 3.81 -2.54) (size 2.286 2.286) (drill 1.4986) (layers "*.Cu" "*.Mask") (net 2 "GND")))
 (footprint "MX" (layer "F.Cu") (at 152.4 133.35)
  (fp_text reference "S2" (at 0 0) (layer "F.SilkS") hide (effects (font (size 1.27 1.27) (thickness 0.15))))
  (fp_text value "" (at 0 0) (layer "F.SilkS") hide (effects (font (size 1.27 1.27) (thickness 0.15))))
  (pad "" np_thru_hole circle (at -5.08 0) (size 1.7018 1.7018) (drill 1.7018) (layers "*.Cu" "*.Mask"))
  (pad "" np_thru_hole circle (at 0 0) (size 3.9878 3.9878) (drill 3.9878) (layers "*.Cu" "*.Mask"))
  (pad "" np_thru_hole circle (at 5.08 0) (size 1.7018 1.7018) (drill 1.7018) (layers "*.Cu" "*.Mask"))
  (pad "1" thru_hole circle (at -2.54 -5.08) (size 2.286 2.286) (drill 1.4986) (layers "*.Cu" "*.Mask") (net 20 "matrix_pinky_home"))
  (pad "1" thru_hole circle (at 2.54 -5.08) (size 2.286 2.286) (drill 1.4986) (layers "*.Cu" "*.Mask") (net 20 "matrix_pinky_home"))
  (pad "2" thru_hole circle (at -3.81 -2.54) (size 2.286 2.286) (drill 1.4986) (layers "*.Cu" "*.Mask") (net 2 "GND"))
  (pad "2" thru_hole circle (at 3.81 -2.54) (size 2.286 2.286) (drill 1.4986) (layers "*.Cu" "*.Mask") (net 2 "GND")))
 (gr_arc (start 255.36083 211.512794) (mid 252.306551 213.23828) (end 248.870324 212.532399) (stroke (width 0.15) (type solid))
  (layer "Edge.Cuts"))
 (gr_line (start 141.9225 107.747172) (end 141.9225 159.404657) (stroke (width 0.15) (type solid)) (layer "Edge.Cuts"))
 (gr_arc (start 180.289795 94.440599) (mid 180.879326 94.333403) (end 181.477446 94.2975) (stroke (width 0.15) (type solid))
  (layer "Edge.Cuts"))
 (gr_arc (start 199.551532 94.2975) (mid 199.923963 94.31139) (end 200.294324 94.352982) (stroke (width 0.15) (type solid))
  (layer "Edge.Cuts"))
 (gr_line (start 145.176799 164.090009) (end 210.048527 188.260368) (stroke (width 0.15) (type solid)) (layer "Edge.Cuts"))
 (gr_line (start 199.551532 94.2975) (end 181.477446 94.2975) (stroke (width 0.15) (type solid)) (layer "Edge.Cuts"))
 (gr_arc (start 141.922501 107.747172) (mid 142.98942 104.659962) (end 145.734849 102.890272) (stroke (width 0.15) (type solid))
  (layer "Edge.Cuts"))
 (gr_line (start 180.289795 94.440599) (end 145.734849 102.890272) (stroke (width 0.15) (type solid)) (layer "Edge.Cuts"))
 (gr_arc (start 210.048528 188.260368) (mid 210.517371 188.462887) (end 210.96311 188.712177) (stroke (width 0.15) (type solid))
  (layer "Edge.Cuts"))
 (gr_arc (start 145.176799 164.090009) (mid 142.81589 162.25698) (end 141.9225 159.404657) (stroke (width 0.15) (type solid))
  (layer "Edge.Cuts"))
 (gr_line (start 210.96311 188.712177) (end 248.870324 212.532399) (stroke (width 0.15) (type solid)) (layer "Edge.Cuts"))
 (gr_arc (start 262.334929 103.673051) (mid 265.345743 105.314473) (end 266.59097 108.509575) (stroke (width 0.15) (type solid))
  (layer "Edge.Cuts"))
 (gr_line (start 262.334929 103.673051) (end 200.294324 94.352982) (stroke (width 0.15) (type solid)) (layer "Edge.Cuts"))
 (gr_line (start 268.437874 193.998943) (end 266.59097 108.509575) (stroke (width 0.15) (type solid)) (layer "Edge.Cuts"))
 (gr_line (start 255.36083 211.512793) (end 267.269263 197.320876) (stroke (width 0.15) (type solid)) (layer "Edge.Cuts"))
 (gr_arc (start 268.437874 193.998944) (mid 268.155699 195.766195) (end 267.269263 197.320876) (stroke (width 0.15) (type solid))
  (layer "Edge.Cuts"))
 (segment (start 259.995 107.49875) (end 259.25185 107.49875) (width 0.25) (layer "B.Cu") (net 16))
 (segment (start 258.2418 108.5088) (end 258.2418 113.3507) (width 0.25) (layer "B.Cu") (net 16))
 (arc (start 258.2418 113.3507) (mid 257.731272 114.583222) (end 256.49875 115.09375) (width 0.25) (layer "B.Cu") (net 16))
 (arc (start 259.25185 107.49875) (mid 258.537637 107.794587) (end 258.2418 108.5088) (width 0.25) (layer "B.Cu") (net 16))
 (segment (start 259.995 110.49875) (end 259.688718 110.49875) (width 0.25) (layer "B.Cu") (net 15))
 (segment (start 258.699 113.168903) (end 258.699857 113.169789) (width 0.25) (layer "B.Cu") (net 15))
 (segment (start 258.699 111.488468) (end 258.699 113.168903) (width 0.25) (layer "B.Cu") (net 15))
 (segment (start 258.699857 113.169789) (end 258.699857 115.432643) (width 0.25) (layer "B.Cu") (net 15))
 (arc (start 259.688718 110.49875) (mid 258.988882 110.788632) (end 258.699 111.488468) (width 0.25) (layer "B.Cu") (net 15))
 (arc (start 258.699857 115.432643) (mid 258.055168 116.989061) (end 256.49875 117.63375) (width 0.25) (layer "B.Cu") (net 15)))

